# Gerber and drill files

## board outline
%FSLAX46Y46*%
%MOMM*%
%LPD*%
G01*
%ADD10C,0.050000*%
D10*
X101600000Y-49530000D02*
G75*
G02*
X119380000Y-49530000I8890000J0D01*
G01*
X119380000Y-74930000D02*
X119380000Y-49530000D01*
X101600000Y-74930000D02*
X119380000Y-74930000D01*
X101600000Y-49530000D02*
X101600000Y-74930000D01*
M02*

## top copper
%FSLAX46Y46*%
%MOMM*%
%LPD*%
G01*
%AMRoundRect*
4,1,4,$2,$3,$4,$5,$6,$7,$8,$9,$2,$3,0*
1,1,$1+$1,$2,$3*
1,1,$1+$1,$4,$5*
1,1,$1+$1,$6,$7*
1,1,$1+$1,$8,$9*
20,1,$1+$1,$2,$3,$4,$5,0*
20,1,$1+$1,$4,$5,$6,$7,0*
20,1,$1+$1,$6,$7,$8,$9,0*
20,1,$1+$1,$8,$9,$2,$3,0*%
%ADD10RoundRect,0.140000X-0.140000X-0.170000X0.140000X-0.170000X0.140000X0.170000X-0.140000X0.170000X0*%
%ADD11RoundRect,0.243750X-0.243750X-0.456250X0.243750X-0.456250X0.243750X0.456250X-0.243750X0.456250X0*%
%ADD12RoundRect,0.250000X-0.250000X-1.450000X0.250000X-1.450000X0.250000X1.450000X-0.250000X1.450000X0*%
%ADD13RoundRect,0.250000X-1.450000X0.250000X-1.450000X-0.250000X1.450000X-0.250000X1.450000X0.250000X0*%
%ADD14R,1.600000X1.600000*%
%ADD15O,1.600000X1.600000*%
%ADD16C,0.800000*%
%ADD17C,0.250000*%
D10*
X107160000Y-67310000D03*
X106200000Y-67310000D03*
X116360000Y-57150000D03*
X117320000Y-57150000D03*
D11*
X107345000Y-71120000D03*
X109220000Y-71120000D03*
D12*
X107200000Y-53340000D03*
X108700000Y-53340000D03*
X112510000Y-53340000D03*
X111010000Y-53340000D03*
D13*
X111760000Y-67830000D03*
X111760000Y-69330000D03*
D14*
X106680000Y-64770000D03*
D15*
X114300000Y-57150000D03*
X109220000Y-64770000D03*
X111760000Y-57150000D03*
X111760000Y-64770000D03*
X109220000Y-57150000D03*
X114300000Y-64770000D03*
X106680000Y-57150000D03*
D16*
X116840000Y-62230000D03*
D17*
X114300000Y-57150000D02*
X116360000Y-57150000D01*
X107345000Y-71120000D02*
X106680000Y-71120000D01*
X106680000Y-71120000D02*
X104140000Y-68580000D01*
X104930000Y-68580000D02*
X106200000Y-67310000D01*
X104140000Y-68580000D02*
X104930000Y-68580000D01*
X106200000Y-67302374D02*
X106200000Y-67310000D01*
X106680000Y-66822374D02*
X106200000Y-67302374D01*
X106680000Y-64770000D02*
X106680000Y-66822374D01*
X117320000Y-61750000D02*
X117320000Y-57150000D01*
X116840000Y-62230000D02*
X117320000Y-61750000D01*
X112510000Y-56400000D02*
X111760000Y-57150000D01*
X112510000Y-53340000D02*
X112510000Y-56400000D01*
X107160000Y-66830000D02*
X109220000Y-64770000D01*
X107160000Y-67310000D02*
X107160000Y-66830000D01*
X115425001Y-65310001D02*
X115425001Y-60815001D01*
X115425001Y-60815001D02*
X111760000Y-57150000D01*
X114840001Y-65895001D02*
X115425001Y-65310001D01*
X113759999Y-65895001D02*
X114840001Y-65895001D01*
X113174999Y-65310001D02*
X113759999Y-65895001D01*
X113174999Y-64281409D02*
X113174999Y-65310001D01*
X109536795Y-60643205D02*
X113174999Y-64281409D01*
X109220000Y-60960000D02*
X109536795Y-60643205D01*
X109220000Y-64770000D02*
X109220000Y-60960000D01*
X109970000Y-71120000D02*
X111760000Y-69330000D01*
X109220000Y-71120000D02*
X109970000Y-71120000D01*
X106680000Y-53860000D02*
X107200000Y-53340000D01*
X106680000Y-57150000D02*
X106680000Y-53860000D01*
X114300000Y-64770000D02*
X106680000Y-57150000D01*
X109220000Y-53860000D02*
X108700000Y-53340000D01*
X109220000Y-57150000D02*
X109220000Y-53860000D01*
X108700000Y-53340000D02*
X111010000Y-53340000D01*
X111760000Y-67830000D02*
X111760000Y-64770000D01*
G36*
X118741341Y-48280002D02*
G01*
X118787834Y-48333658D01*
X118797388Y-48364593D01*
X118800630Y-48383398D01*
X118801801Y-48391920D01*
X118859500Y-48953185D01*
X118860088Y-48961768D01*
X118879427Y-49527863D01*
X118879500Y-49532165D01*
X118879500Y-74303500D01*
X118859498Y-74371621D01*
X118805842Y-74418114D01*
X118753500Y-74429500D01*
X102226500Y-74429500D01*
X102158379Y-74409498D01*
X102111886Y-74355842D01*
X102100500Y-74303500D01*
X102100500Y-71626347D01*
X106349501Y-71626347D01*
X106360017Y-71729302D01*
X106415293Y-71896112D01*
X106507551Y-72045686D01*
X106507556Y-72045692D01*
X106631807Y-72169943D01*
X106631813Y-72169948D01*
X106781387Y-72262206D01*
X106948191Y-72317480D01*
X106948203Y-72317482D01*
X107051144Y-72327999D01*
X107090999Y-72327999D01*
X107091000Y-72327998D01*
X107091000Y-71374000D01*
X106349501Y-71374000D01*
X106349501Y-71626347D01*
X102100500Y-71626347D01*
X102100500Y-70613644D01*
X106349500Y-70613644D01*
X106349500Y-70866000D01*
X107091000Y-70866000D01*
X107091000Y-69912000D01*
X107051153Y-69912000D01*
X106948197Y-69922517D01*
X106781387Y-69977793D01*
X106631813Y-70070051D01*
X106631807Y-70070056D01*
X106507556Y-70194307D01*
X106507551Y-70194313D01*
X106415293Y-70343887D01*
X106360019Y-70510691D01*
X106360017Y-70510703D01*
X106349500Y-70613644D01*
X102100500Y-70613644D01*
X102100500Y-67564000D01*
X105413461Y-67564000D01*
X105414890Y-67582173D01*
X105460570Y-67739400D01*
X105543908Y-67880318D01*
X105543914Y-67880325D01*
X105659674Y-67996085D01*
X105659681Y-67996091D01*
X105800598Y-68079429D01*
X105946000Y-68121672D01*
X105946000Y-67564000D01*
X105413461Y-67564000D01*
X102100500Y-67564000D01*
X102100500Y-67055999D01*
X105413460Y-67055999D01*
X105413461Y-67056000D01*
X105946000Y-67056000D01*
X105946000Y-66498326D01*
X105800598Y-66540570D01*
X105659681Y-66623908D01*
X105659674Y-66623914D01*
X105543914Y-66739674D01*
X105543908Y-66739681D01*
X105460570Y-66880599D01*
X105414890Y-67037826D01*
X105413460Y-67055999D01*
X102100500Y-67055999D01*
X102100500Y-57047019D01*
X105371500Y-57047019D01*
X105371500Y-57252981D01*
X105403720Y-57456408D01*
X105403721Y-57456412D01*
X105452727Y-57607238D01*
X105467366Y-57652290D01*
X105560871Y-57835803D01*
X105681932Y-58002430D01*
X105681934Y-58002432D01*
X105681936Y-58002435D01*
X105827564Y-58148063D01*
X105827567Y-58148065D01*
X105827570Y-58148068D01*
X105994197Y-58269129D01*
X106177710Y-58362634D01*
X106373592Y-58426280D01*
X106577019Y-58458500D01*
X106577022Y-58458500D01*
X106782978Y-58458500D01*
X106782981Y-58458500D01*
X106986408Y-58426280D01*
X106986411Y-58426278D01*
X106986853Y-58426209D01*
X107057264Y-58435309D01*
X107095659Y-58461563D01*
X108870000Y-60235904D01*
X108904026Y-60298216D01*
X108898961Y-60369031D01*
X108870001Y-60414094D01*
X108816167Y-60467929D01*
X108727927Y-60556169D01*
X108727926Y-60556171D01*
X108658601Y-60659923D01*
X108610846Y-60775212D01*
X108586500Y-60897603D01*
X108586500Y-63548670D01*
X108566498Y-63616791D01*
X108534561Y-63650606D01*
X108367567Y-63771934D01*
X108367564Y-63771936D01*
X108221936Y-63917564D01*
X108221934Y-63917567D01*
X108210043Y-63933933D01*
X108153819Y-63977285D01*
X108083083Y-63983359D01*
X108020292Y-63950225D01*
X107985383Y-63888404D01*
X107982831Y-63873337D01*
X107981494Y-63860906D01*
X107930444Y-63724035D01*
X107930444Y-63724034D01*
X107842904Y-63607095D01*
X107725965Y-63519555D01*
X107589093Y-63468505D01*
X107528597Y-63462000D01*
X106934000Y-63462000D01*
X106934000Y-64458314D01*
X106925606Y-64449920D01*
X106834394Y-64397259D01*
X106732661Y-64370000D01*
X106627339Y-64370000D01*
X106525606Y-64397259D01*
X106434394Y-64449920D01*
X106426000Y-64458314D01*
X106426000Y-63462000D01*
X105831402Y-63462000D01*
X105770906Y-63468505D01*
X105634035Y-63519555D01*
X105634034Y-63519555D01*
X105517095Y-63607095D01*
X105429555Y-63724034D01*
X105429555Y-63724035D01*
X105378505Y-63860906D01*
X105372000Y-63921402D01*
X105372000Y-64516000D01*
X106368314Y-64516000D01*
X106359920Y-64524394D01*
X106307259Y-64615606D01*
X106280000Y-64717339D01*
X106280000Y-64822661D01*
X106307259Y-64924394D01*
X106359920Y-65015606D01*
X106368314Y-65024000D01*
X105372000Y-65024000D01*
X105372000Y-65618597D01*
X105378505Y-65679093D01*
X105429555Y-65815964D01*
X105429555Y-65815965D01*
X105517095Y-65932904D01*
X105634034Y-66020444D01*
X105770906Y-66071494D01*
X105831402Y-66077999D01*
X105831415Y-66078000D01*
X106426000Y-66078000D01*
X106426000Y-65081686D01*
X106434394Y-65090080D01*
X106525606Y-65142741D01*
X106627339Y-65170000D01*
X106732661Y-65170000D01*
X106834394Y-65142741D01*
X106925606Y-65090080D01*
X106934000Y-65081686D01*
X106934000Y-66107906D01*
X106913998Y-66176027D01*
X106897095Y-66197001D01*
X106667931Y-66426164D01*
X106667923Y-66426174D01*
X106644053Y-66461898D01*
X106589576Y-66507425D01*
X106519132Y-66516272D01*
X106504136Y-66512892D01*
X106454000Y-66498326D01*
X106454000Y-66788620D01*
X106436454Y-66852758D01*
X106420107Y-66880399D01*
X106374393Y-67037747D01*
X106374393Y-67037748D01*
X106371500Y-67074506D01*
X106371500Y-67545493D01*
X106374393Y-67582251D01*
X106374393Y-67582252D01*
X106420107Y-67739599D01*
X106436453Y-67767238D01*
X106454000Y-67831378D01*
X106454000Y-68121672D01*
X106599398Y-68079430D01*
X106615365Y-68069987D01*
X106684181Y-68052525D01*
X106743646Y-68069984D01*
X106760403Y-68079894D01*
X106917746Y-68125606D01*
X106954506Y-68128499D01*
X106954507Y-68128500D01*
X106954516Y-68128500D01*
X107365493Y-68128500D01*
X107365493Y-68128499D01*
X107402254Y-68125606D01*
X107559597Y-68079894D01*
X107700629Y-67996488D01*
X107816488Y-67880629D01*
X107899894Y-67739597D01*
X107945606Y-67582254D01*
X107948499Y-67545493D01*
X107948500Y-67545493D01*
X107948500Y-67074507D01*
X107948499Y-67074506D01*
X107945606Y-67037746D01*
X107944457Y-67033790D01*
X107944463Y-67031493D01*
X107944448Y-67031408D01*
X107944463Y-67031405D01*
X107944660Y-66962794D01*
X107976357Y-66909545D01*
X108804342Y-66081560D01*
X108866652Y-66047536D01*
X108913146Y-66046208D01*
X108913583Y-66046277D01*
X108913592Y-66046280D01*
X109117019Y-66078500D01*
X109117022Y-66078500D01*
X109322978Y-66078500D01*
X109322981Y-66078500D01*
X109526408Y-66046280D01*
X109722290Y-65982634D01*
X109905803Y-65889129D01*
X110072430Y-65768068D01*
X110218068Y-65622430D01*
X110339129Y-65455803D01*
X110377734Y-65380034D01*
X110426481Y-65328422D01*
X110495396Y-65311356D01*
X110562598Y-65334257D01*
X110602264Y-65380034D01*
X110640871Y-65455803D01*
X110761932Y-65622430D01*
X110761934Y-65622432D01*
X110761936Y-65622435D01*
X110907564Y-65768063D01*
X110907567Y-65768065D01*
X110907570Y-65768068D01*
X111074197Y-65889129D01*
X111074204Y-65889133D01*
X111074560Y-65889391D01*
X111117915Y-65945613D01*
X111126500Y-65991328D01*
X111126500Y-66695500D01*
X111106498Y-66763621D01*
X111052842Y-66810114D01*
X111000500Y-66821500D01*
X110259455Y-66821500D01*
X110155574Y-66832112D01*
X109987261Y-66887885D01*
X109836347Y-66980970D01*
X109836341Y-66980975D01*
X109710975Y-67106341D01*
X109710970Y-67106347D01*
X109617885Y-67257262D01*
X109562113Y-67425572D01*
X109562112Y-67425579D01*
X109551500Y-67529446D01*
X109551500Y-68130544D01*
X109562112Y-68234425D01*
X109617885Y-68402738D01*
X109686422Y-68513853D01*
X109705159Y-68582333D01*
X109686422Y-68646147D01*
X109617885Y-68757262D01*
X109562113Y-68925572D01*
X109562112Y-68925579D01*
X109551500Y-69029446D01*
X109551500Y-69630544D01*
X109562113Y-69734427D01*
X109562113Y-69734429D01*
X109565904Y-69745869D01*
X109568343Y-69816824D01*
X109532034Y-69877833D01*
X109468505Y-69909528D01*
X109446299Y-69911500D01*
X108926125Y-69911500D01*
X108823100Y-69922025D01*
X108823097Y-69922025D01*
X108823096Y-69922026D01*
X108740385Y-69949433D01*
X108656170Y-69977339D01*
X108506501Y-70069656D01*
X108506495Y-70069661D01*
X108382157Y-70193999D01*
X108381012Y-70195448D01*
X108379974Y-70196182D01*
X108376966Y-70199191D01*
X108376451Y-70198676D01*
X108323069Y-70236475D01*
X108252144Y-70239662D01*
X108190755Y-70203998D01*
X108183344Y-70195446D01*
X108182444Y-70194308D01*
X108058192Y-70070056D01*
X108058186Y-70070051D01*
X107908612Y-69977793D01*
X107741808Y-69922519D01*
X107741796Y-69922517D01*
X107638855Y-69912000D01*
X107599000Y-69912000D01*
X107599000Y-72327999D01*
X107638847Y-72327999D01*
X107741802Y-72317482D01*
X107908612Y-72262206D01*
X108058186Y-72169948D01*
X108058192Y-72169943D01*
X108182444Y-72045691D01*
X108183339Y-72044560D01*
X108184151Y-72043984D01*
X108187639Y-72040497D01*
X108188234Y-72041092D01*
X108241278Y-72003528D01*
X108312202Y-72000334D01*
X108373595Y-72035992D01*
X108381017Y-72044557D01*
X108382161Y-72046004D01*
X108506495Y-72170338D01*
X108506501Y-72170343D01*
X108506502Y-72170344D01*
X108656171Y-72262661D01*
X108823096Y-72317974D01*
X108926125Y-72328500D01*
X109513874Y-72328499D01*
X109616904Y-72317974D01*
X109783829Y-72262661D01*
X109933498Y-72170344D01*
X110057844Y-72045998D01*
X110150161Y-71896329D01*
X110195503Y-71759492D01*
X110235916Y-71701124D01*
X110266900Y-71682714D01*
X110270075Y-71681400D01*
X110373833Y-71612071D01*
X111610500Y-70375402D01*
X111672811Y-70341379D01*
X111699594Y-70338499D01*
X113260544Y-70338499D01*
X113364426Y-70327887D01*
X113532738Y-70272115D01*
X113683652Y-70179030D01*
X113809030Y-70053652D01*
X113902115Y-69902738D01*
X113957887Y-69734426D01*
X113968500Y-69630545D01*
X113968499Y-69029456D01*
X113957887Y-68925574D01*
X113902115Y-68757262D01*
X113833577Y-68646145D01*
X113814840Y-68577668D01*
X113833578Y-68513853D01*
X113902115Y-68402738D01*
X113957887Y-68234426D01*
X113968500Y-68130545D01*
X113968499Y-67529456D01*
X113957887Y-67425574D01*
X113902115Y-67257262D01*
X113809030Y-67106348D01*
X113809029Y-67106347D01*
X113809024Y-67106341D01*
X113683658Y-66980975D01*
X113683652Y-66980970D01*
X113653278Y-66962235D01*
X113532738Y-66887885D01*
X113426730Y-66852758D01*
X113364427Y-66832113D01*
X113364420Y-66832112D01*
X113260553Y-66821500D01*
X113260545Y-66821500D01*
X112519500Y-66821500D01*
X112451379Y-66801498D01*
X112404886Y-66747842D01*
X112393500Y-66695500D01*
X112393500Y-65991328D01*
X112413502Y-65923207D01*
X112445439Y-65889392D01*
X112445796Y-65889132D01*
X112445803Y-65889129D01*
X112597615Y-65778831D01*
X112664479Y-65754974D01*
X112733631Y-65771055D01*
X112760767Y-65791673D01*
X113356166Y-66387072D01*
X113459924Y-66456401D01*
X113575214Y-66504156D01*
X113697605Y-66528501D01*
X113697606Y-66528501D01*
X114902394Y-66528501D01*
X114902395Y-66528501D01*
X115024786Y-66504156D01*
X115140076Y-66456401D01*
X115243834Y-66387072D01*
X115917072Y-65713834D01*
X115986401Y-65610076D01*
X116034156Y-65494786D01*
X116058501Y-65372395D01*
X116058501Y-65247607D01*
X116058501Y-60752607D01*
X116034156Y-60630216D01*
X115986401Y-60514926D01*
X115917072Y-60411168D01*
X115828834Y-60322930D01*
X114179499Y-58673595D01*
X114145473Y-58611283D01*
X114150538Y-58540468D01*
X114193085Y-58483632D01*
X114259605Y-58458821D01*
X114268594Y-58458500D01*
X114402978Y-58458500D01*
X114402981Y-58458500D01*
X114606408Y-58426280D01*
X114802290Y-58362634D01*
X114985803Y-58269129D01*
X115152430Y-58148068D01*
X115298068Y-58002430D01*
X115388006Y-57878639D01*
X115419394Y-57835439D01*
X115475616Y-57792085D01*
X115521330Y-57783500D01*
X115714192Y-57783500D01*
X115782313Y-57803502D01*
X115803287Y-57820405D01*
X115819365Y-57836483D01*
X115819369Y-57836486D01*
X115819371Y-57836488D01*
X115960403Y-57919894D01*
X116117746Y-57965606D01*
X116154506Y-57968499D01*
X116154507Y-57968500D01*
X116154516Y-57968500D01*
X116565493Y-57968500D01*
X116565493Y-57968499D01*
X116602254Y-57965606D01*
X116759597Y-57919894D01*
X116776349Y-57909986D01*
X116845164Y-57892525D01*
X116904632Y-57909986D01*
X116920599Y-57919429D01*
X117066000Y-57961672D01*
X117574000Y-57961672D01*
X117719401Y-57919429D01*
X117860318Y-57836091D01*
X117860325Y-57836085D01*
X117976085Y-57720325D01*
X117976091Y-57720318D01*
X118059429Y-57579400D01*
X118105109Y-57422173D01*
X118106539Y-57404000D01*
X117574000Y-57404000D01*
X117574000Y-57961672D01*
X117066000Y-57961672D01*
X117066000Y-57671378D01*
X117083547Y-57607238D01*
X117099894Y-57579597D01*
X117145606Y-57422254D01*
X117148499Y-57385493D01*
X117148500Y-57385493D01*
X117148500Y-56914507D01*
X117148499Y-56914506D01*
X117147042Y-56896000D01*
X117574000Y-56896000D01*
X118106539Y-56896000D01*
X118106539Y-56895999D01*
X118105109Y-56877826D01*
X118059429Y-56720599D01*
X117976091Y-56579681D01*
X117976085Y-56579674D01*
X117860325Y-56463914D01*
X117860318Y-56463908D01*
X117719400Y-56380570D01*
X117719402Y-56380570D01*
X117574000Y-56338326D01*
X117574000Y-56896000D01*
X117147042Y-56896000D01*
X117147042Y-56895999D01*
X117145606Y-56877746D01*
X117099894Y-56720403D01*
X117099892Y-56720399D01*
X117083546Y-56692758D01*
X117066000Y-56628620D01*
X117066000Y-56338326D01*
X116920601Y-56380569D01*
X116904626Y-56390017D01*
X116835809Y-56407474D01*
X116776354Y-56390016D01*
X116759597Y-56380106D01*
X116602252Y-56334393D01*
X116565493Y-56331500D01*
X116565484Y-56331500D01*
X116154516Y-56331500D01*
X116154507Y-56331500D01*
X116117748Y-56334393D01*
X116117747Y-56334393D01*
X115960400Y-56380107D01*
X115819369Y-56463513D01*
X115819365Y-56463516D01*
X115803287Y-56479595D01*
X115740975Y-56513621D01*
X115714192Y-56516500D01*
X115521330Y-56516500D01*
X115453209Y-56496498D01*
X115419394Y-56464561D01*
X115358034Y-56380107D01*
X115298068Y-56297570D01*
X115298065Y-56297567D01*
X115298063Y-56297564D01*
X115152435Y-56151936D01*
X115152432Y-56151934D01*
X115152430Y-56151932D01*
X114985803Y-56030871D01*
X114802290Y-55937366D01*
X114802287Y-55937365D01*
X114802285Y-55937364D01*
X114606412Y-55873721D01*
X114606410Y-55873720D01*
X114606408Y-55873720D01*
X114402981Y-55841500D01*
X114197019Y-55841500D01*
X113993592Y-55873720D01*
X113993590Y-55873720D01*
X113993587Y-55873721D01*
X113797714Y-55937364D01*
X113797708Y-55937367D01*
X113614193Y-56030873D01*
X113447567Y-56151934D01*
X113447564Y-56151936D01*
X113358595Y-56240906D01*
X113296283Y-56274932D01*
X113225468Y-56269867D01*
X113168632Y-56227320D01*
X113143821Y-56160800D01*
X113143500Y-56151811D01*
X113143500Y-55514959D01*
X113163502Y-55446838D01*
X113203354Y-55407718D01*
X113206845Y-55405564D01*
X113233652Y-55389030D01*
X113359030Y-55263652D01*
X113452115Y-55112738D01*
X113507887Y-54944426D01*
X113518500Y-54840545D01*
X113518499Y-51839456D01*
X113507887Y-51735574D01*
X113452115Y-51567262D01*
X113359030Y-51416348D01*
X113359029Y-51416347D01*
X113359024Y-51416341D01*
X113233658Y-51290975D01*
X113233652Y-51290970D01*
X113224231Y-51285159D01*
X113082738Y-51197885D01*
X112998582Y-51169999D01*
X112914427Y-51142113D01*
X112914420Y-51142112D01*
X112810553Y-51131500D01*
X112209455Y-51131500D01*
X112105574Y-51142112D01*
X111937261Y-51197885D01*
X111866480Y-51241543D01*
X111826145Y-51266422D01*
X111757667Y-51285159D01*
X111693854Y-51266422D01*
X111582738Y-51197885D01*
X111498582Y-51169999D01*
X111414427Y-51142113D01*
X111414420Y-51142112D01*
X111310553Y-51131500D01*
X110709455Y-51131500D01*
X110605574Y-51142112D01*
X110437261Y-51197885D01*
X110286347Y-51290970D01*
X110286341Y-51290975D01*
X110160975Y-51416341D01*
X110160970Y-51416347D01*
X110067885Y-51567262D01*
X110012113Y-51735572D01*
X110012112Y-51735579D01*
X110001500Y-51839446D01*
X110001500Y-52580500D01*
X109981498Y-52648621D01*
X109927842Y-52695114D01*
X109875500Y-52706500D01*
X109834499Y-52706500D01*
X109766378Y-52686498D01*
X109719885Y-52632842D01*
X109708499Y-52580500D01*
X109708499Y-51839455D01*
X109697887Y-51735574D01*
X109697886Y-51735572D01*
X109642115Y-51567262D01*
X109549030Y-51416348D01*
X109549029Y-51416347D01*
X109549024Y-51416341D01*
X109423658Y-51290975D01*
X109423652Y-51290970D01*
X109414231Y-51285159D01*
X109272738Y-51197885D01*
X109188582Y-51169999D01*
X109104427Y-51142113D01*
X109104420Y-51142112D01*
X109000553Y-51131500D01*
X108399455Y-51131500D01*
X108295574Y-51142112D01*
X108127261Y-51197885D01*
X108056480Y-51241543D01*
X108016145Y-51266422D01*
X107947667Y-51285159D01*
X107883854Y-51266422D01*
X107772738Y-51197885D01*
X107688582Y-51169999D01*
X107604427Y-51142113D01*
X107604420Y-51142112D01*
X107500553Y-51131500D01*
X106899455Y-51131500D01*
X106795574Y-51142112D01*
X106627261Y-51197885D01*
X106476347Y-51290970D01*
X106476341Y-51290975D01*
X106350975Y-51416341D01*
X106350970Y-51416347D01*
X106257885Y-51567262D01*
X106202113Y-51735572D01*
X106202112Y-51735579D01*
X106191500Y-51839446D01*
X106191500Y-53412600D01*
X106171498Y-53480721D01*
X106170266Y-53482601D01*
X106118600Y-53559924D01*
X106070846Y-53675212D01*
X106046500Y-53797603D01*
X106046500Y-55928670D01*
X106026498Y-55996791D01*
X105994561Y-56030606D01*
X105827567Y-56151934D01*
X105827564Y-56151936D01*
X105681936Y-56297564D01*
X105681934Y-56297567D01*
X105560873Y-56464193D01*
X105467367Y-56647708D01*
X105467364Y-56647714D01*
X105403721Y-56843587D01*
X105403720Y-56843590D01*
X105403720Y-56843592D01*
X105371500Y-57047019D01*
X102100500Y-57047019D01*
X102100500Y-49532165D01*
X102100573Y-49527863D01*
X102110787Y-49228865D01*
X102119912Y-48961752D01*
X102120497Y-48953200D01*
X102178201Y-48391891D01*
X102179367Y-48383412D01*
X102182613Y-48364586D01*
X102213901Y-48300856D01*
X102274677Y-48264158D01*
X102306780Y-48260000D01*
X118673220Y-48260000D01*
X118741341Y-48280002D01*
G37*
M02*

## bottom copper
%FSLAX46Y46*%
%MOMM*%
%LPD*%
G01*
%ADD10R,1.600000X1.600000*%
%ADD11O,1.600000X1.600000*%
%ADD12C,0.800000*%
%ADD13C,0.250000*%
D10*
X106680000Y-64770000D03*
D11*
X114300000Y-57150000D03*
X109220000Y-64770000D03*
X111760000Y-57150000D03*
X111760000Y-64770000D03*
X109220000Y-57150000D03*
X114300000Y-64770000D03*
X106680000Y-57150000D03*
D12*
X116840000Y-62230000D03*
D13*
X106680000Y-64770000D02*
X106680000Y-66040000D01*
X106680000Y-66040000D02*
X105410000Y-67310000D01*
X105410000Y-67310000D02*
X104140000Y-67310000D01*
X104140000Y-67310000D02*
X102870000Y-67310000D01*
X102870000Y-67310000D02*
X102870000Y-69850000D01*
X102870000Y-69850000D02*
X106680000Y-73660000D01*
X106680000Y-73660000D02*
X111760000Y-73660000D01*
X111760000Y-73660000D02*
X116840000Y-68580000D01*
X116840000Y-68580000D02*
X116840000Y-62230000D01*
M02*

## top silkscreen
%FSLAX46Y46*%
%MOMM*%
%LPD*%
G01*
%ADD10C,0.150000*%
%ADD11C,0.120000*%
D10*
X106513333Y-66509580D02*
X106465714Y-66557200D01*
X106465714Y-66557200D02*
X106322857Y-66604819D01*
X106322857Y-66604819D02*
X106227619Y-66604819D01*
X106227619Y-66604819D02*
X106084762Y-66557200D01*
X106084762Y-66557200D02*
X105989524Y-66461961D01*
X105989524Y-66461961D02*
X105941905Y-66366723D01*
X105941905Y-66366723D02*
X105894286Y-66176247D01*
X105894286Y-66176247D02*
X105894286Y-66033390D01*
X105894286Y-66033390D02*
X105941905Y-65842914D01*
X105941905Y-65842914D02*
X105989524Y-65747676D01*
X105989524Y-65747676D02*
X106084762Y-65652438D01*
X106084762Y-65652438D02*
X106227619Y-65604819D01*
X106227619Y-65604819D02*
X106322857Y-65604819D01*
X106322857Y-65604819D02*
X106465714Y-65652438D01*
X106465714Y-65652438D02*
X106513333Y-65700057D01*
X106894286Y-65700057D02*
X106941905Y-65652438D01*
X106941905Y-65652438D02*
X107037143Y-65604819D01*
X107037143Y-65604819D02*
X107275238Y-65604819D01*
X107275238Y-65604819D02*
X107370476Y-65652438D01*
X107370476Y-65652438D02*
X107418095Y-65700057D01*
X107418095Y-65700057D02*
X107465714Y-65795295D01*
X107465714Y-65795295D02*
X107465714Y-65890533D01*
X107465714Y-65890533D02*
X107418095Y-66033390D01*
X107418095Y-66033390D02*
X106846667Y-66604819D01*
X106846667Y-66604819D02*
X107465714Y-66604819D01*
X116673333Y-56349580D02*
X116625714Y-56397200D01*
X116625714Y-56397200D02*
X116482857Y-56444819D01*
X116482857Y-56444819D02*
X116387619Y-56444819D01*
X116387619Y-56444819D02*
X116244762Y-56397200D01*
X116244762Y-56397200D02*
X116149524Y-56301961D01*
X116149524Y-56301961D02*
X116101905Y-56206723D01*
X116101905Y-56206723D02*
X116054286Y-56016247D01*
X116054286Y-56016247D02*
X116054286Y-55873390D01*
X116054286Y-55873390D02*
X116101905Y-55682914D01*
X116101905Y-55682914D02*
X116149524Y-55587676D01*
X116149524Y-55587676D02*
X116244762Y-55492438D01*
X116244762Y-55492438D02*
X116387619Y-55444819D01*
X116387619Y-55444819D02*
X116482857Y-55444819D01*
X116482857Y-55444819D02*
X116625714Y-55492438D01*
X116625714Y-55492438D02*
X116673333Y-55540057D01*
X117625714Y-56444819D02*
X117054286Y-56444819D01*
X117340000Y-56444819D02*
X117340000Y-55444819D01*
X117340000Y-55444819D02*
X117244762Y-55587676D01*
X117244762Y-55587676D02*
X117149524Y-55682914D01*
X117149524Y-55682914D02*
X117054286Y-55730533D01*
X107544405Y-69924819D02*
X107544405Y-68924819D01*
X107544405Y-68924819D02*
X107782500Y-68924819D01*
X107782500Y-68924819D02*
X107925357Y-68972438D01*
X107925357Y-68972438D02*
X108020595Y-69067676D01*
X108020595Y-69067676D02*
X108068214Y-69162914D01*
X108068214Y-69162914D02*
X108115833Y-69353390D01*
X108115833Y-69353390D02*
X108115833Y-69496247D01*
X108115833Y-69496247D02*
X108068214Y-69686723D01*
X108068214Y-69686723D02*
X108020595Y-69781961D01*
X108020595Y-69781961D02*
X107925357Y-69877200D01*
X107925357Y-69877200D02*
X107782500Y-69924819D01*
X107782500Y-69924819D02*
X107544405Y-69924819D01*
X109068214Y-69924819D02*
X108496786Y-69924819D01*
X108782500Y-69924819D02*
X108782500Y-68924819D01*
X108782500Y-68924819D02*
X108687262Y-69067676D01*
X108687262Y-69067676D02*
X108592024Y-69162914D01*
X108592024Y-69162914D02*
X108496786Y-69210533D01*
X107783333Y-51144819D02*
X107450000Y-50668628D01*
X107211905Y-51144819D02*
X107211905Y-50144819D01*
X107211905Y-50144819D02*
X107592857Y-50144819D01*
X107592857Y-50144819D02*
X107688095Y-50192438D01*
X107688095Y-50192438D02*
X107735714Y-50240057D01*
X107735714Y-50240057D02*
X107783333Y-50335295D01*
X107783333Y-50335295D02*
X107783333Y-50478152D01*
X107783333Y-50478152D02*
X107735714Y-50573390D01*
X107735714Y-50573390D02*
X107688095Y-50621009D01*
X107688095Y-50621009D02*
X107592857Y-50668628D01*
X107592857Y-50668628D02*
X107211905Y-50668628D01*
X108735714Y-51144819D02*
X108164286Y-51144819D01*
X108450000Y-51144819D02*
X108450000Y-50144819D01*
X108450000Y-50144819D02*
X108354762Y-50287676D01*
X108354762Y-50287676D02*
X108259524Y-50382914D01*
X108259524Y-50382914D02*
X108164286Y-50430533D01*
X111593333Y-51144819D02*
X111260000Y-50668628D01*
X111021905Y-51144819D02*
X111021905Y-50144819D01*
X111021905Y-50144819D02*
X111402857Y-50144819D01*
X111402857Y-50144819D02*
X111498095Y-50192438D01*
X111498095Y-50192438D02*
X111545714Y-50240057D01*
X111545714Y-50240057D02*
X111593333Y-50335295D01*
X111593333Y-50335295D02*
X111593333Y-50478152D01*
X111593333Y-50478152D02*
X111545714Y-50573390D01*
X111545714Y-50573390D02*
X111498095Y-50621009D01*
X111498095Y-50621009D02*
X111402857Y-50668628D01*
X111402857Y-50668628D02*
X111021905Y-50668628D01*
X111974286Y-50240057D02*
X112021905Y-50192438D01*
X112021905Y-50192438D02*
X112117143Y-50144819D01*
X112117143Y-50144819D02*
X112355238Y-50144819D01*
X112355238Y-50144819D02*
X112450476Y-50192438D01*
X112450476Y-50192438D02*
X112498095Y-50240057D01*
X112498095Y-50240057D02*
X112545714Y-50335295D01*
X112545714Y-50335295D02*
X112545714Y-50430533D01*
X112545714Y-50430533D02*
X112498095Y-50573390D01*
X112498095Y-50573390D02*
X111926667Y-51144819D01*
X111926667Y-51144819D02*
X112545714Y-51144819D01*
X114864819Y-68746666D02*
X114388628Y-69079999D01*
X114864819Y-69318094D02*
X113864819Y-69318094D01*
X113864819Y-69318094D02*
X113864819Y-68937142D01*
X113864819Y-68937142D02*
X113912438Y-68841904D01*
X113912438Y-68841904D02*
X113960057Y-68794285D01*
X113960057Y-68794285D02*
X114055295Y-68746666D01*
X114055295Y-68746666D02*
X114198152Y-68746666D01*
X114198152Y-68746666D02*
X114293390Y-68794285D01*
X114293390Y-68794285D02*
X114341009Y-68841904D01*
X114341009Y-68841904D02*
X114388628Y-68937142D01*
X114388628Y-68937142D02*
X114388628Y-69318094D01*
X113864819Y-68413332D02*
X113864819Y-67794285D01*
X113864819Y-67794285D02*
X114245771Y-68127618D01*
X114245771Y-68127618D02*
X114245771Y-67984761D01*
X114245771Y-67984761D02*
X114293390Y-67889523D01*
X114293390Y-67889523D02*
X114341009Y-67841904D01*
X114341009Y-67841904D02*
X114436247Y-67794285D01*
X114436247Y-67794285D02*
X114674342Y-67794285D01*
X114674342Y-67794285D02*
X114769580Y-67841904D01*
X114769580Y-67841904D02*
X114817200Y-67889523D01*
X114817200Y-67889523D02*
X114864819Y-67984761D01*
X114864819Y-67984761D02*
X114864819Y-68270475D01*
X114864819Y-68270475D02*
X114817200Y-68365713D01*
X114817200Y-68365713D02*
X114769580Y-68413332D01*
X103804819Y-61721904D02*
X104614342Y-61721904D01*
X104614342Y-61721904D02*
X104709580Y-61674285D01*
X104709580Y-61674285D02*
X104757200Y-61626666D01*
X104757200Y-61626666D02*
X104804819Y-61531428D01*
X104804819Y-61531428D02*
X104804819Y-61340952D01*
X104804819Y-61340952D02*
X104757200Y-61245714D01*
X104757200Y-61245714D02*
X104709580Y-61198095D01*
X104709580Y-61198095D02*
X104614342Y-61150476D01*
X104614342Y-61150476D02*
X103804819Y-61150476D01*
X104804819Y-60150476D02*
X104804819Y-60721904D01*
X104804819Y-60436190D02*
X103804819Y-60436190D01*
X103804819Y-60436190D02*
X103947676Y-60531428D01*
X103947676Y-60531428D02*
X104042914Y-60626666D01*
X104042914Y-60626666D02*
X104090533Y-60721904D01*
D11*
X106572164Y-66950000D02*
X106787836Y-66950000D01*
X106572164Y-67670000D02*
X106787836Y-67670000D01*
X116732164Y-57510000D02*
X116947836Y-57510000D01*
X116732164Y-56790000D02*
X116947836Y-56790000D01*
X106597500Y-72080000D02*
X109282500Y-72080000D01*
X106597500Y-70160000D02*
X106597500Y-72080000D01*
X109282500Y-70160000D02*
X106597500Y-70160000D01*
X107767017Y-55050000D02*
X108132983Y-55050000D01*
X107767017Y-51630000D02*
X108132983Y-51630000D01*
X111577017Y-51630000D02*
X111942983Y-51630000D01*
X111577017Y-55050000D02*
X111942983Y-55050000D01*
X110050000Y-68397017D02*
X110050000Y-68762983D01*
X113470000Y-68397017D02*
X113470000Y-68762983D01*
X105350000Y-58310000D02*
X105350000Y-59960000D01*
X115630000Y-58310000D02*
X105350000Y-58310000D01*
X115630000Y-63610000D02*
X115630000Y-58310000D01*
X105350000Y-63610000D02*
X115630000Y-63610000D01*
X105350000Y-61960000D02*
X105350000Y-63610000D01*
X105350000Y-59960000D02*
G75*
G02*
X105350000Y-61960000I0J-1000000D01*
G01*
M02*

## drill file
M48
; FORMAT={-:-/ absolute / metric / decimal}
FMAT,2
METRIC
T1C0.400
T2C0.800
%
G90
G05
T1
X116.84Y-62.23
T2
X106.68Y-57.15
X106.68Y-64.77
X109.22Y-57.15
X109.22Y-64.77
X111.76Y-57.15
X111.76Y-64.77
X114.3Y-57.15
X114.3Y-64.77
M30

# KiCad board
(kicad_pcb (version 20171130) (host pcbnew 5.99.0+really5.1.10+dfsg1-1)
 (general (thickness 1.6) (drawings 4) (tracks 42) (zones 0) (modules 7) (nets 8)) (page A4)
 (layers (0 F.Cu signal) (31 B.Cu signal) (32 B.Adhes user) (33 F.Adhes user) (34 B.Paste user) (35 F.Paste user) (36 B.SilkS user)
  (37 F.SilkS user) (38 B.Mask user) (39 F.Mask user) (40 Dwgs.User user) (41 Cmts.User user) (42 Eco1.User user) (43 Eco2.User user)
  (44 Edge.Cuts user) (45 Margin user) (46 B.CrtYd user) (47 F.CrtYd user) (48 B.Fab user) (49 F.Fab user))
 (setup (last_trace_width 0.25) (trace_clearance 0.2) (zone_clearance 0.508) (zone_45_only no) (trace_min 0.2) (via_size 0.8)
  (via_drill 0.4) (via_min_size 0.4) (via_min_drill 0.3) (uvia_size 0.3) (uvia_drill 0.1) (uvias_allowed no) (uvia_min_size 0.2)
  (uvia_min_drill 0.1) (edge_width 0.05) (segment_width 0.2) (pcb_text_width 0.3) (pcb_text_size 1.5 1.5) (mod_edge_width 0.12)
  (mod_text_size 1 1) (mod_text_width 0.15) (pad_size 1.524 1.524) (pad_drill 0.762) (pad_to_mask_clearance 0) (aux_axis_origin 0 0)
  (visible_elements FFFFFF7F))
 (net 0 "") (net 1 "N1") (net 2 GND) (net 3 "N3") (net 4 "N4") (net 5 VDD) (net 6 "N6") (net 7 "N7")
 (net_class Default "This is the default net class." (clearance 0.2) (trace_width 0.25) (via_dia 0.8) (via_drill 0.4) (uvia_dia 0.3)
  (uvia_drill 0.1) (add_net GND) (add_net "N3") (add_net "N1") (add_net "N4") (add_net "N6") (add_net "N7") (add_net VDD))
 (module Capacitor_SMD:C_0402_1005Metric (layer F.Cu) (at 106.68 67.31)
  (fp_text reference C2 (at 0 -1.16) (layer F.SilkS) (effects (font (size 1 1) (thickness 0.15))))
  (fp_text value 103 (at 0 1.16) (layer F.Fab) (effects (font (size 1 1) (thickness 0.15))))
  (fp_line (start -0.107836 -0.36) (end 0.107836 -0.36) (layer F.SilkS) (width 0.12))
  (fp_line (start -0.107836 0.36) (end 0.107836 0.36) (layer F.SilkS) (width 0.12))
  (pad 2 smd roundrect (at 0.48 0) (size 0.56 0.62) (layers F.Cu F.Paste F.Mask) (roundrect_rratio 0.25) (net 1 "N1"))
  (pad 1 smd roundrect (at -0.48 0) (size 0.56 0.62) (layers F.Cu F.Paste F.Mask) (roundrect_rratio 0.25) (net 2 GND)))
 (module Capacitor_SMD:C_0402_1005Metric (layer F.Cu) (at 116.84 57.15)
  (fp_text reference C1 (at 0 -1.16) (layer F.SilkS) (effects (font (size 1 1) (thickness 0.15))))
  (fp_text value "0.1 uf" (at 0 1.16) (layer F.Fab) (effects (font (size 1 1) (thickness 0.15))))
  (fp_line (start -0.107836 0.36) (end 0.107836 0.36) (layer F.SilkS) (width 0.12))
  (fp_line (start -0.107836 -0.36) (end 0.107836 -0.36) (layer F.SilkS) (width 0.12))
  (pad 1 smd roundrect (at -0.48 0) (size 0.56 0.62) (layers F.Cu F.Paste F.Mask) (roundrect_rratio 0.25) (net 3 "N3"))
  (pad 2 smd roundrect (at 0.48 0) (size 0.56 0.62) (layers F.Cu F.Paste F.Mask) (roundrect_rratio 0.25) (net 2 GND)))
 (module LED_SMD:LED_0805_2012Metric (layer F.Cu) (at 108.2825 71.12)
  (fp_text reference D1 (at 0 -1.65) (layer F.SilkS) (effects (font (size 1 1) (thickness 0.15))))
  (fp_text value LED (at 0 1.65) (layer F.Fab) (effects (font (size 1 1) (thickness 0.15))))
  (fp_line (start -1.685 0.96) (end 1 0.96) (layer F.SilkS) (width 0.12))
  (fp_line (start -1.685 -0.96) (end -1.685 0.96) (layer F.SilkS) (width 0.12))
  (fp_line (start 1 -0.96) (end -1.685 -0.96) (layer F.SilkS) (width 0.12))
  (pad 1 smd roundrect (at -0.9375 0) (size 0.975 1.4) (layers F.Cu F.Paste F.Mask) (roundrect_rratio 0.25) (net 2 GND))
  (pad 2 smd roundrect (at 0.9375 0) (size 0.975 1.4) (layers F.Cu F.Paste F.Mask) (roundrect_rratio 0.25) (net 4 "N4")))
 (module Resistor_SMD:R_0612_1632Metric (layer F.Cu) (at 107.95 53.34)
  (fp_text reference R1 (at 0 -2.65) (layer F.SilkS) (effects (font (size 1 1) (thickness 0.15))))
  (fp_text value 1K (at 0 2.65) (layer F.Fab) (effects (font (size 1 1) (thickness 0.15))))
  (fp_line (start -0.182983 1.71) (end 0.182983 1.71) (layer F.SilkS) (width 0.12))
  (fp_line (start -0.182983 -1.71) (end 0.182983 -1.71) (layer F.SilkS) (width 0.12))
  (pad 1 smd roundrect (at -0.75 0) (size 1 3.4) (layers F.Cu F.Paste F.Mask) (roundrect_rratio 0.25) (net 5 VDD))
  (pad 2 smd roundrect (at 0.75 0) (size 1 3.4) (layers F.Cu F.Paste F.Mask) (roundrect_rratio 0.25) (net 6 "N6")))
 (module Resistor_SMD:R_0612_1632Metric (layer F.Cu) (at 111.76 53.34)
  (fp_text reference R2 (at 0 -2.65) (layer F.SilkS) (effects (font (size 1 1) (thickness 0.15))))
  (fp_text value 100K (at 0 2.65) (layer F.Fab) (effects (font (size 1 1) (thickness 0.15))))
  (fp_line (start -0.182983 -1.71) (end 0.182983 -1.71) (layer F.SilkS) (width 0.12))
  (fp_line (start -0.182983 1.71) (end 0.182983 1.71) (layer F.SilkS) (width 0.12))
  (pad 2 smd roundrect (at 0.75 0) (size 1 3.4) (layers F.Cu F.Paste F.Mask) (roundrect_rratio 0.25) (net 1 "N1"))
  (pad 1 smd roundrect (at -0.75 0) (size 1 3.4) (layers F.Cu F.Paste F.Mask) (roundrect_rratio 0.25) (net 6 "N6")))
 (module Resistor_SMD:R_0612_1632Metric (layer F.Cu) (at 111.76 68.58 270)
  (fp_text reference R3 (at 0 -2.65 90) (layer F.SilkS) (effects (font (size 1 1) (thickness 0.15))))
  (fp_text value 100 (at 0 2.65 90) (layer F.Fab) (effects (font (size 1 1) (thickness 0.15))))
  (fp_line (start -0.182983 1.71) (end 0.182983 1.71) (layer F.SilkS) (width 0.12))
  (fp_line (start -0.182983 -1.71) (end 0.182983 -1.71) (layer F.SilkS) (width 0.12))
  (pad 1 smd roundrect (at -0.75 0 270) (size 1 3.4) (layers F.Cu F.Paste F.Mask) (roundrect_rratio 0.25) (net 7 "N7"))
  (pad 2 smd roundrect (at 0.75 0 270) (size 1 3.4) (layers F.Cu F.Paste F.Mask) (roundrect_rratio 0.25) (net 4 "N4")))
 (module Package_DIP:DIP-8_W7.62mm (layer F.Cu) (at 106.68 64.77 90)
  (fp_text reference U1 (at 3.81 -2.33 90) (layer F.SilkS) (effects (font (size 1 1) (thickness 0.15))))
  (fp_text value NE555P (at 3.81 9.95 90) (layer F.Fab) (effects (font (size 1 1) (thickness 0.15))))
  (fp_line (start 6.46 -1.33) (end 4.81 -1.33) (layer F.SilkS) (width 0.12))
  (fp_line (start 6.46 8.95) (end 6.46 -1.33) (layer F.SilkS) (width 0.12))
  (fp_line (start 1.16 8.95) (end 6.46 8.95) (layer F.SilkS) (width 0.12))
  (fp_line (start 1.16 -1.33) (end 1.16 8.95) (layer F.SilkS) (width 0.12))
  (fp_line (start 2.81 -1.33) (end 1.16 -1.33) (layer F.SilkS) (width 0.12))
  (fp_arc (start 3.81 -1.33) (end 2.81 -1.33) (angle -180) (layer F.SilkS) (width 0.12))
  (pad 1 thru_hole rect (at 0 0 90) (size 1.6 1.6) (drill 0.8) (layers *.Cu *.Mask) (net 2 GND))
  (pad 5 thru_hole oval (at 7.62 7.62 90) (size 1.6 1.6) (drill 0.8) (layers *.Cu *.Mask) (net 3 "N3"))
  (pad 2 thru_hole oval (at 0 2.54 90) (size 1.6 1.6) (drill 0.8) (layers *.Cu *.Mask) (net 1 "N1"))
  (pad 6 thru_hole oval (at 7.62 5.08 90) (size 1.6 1.6) (drill 0.8) (layers *.Cu *.Mask) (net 1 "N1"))
  (pad 3 thru_hole oval (at 0 5.08 90) (size 1.6 1.6) (drill 0.8) (layers *.Cu *.Mask) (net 7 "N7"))
  (pad 7 thru_hole oval (at 7.62 2.54 90) (size 1.6 1.6) (drill 0.8) (layers *.Cu *.Mask) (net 6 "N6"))
  (pad 4 thru_hole oval (at 0 7.62 90) (size 1.6 1.6) (drill 0.8) (layers *.Cu *.Mask) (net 5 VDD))
  (pad 8 thru_hole oval (at 7.62 0 90) (size 1.6 1.6) (drill 0.8) (layers *.Cu *.Mask) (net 5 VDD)))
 (gr_arc (start 110.49 49.53) (end 119.38 49.53) (angle -180) (layer Edge.Cuts) (width 0.05))
 (gr_line (start 119.38 74.93) (end 119.38 49.53) (layer Edge.Cuts) (width 0.05))
 (gr_line (start 101.6 74.93) (end 119.38 74.93) (layer Edge.Cuts) (width 0.05))
 (gr_line (start 101.6 49.53) (end 101.6 74.93) (layer Edge.Cuts) (width 0.05))
 (segment (start 114.3 57.15) (end 116.36 57.15) (width 0.25) (layer F.Cu) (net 3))
 (segment (start 107.345 71.12) (end 106.68 71.12) (width 0.25) (layer F.Cu) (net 2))
 (segment (start 106.68 71.12) (end 104.14 68.58) (width 0.25) (layer F.Cu) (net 2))
 (segment (start 104.93 68.58) (end 106.2 67.31) (width 0.25) (layer F.Cu) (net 2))
 (segment (start 104.14 68.58) (end 104.93 68.58) (width 0.25) (layer F.Cu) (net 2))
 (segment (start 106.2 67.302374) (end 106.2 67.31) (width 0.25) (layer F.Cu) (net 2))
 (segment (start 106.68 66.822374) (end 106.2 67.302374) (width 0.25) (layer F.Cu) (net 2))
 (segment (start 106.68 64.77) (end 106.68 66.822374) (width 0.25) (layer F.Cu) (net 2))
 (segment (start 106.68 64.77) (end 106.68 66.04) (width 0.25) (layer B.Cu) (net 2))
 (segment (start 106.68 66.04) (end 105.41 67.31) (width 0.25) (layer B.Cu) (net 2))
 (segment (start 105.41 67.31) (end 104.14 67.31) (width 0.25) (layer B.Cu) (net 2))
 (segment (start 104.14 67.31) (end 102.87 67.31) (width 0.25) (layer B.Cu) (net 2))
 (segment (start 102.87 67.31) (end 102.87 69.85) (width 0.25) (layer B.Cu) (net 2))
 (segment (start 102.87 69.85) (end 106.68 73.66) (width 0.25) (layer B.Cu) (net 2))
 (segment (start 106.68 73.66) (end 111.76 73.66) (width 0.25) (layer B.Cu) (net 2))
 (segment (start 111.76 73.66) (end 116.84 68.58) (width 0.25) (layer B.Cu) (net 2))
 (via (at 116.84 62.23) (size 0.8) (drill 0.4) (layers F.Cu B.Cu) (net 2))
 (segment (start 116.84 68.58) (end 116.84 62.23) (width 0.25) (layer B.Cu) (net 2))
 (segment (start 117.32 61.75) (end 117.32 57.15) (width 0.25) (layer F.Cu) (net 2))
 (segment (start 116.84 62.23) (end 117.32 61.75) (width 0.25) (layer F.Cu) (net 2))
 (segment (start 112.51 56.4) (end 111.76 57.15) (width 0.25) (layer F.Cu) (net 1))
 (segment (start 112.51 53.34) (end 112.51 56.4) (width 0.25) (layer F.Cu) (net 1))
 (segment (start 107.16 66.83) (end 109.22 64.77) (width 0.25) (layer F.Cu) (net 1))
 (segment (start 107.16 67.31) (end 107.16 66.83) (width 0.25) (layer F.Cu) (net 1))
 (segment (start 115.425001 65.310001) (end 115.425001 60.815001) (width 0.25) (layer F.Cu) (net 1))
 (segment (start 115.425001 60.815001) (end 111.76 57.15) (width 0.25) (layer F.Cu) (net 1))
 (segment (start 114.840001 65.895001) (end 115.425001 65.310001) (width 0.25) (layer F.Cu) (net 1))
 (segment (start 113.759999 65.895001) (end 114.840001 65.895001) (width 0.25) (layer F.Cu) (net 1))
 (segment (start 113.174999 65.310001) (end 113.759999 65.895001) (width 0.25) (layer F.Cu) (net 1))
 (segment (start 113.174999 64.281409) (end 113.174999 65.310001) (width 0.25) (layer F.Cu) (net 1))
 (segment (start 109.536795 60.643205) (end 113.174999 64.281409) (width 0.25) (layer F.Cu) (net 1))
 (segment (start 109.22 60.96) (end 109.536795 60.643205) (width 0.25) (layer F.Cu) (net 1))
 (segment (start 109.22 64.77) (end 109.22 60.96) (width 0.25) (layer F.Cu) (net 1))
 (segment (start 109.97 71.12) (end 111.76 69.33) (width 0.25) (layer F.Cu) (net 4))
 (segment (start 109.22 71.12) (end 109.97 71.12) (width 0.25) (layer F.Cu) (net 4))
 (segment (start 106.68 53.86) (end 107.2 53.34) (width 0.25) (layer F.Cu) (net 5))
 (segment (start 106.68 57.15) (end 106.68 53.86) (width 0.25) (layer F.Cu) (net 5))
 (segment (start 114.3 64.77) (end 106.68 57.15) (width 0.25) (layer F.Cu) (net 5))
 (segment (start 109.22 53.86) (end 108.7 53.34) (width 0.25) (layer F.Cu) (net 6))
 (segment (start 109.22 57.15) (end 109.22 53.86) (width 0.25) (layer F.Cu) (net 6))
 (segment (start 108.7 53.34) (end 111.01 53.34) (width 0.25) (layer F.Cu) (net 6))
 (segment (start 111.76 67.83) (end 111.76 64.77) (width 0.25) (layer F.Cu) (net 7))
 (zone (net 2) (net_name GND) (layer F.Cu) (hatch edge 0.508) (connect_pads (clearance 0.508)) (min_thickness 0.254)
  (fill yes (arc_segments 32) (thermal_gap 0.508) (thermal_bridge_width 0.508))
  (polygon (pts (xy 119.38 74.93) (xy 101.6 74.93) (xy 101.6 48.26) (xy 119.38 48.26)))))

